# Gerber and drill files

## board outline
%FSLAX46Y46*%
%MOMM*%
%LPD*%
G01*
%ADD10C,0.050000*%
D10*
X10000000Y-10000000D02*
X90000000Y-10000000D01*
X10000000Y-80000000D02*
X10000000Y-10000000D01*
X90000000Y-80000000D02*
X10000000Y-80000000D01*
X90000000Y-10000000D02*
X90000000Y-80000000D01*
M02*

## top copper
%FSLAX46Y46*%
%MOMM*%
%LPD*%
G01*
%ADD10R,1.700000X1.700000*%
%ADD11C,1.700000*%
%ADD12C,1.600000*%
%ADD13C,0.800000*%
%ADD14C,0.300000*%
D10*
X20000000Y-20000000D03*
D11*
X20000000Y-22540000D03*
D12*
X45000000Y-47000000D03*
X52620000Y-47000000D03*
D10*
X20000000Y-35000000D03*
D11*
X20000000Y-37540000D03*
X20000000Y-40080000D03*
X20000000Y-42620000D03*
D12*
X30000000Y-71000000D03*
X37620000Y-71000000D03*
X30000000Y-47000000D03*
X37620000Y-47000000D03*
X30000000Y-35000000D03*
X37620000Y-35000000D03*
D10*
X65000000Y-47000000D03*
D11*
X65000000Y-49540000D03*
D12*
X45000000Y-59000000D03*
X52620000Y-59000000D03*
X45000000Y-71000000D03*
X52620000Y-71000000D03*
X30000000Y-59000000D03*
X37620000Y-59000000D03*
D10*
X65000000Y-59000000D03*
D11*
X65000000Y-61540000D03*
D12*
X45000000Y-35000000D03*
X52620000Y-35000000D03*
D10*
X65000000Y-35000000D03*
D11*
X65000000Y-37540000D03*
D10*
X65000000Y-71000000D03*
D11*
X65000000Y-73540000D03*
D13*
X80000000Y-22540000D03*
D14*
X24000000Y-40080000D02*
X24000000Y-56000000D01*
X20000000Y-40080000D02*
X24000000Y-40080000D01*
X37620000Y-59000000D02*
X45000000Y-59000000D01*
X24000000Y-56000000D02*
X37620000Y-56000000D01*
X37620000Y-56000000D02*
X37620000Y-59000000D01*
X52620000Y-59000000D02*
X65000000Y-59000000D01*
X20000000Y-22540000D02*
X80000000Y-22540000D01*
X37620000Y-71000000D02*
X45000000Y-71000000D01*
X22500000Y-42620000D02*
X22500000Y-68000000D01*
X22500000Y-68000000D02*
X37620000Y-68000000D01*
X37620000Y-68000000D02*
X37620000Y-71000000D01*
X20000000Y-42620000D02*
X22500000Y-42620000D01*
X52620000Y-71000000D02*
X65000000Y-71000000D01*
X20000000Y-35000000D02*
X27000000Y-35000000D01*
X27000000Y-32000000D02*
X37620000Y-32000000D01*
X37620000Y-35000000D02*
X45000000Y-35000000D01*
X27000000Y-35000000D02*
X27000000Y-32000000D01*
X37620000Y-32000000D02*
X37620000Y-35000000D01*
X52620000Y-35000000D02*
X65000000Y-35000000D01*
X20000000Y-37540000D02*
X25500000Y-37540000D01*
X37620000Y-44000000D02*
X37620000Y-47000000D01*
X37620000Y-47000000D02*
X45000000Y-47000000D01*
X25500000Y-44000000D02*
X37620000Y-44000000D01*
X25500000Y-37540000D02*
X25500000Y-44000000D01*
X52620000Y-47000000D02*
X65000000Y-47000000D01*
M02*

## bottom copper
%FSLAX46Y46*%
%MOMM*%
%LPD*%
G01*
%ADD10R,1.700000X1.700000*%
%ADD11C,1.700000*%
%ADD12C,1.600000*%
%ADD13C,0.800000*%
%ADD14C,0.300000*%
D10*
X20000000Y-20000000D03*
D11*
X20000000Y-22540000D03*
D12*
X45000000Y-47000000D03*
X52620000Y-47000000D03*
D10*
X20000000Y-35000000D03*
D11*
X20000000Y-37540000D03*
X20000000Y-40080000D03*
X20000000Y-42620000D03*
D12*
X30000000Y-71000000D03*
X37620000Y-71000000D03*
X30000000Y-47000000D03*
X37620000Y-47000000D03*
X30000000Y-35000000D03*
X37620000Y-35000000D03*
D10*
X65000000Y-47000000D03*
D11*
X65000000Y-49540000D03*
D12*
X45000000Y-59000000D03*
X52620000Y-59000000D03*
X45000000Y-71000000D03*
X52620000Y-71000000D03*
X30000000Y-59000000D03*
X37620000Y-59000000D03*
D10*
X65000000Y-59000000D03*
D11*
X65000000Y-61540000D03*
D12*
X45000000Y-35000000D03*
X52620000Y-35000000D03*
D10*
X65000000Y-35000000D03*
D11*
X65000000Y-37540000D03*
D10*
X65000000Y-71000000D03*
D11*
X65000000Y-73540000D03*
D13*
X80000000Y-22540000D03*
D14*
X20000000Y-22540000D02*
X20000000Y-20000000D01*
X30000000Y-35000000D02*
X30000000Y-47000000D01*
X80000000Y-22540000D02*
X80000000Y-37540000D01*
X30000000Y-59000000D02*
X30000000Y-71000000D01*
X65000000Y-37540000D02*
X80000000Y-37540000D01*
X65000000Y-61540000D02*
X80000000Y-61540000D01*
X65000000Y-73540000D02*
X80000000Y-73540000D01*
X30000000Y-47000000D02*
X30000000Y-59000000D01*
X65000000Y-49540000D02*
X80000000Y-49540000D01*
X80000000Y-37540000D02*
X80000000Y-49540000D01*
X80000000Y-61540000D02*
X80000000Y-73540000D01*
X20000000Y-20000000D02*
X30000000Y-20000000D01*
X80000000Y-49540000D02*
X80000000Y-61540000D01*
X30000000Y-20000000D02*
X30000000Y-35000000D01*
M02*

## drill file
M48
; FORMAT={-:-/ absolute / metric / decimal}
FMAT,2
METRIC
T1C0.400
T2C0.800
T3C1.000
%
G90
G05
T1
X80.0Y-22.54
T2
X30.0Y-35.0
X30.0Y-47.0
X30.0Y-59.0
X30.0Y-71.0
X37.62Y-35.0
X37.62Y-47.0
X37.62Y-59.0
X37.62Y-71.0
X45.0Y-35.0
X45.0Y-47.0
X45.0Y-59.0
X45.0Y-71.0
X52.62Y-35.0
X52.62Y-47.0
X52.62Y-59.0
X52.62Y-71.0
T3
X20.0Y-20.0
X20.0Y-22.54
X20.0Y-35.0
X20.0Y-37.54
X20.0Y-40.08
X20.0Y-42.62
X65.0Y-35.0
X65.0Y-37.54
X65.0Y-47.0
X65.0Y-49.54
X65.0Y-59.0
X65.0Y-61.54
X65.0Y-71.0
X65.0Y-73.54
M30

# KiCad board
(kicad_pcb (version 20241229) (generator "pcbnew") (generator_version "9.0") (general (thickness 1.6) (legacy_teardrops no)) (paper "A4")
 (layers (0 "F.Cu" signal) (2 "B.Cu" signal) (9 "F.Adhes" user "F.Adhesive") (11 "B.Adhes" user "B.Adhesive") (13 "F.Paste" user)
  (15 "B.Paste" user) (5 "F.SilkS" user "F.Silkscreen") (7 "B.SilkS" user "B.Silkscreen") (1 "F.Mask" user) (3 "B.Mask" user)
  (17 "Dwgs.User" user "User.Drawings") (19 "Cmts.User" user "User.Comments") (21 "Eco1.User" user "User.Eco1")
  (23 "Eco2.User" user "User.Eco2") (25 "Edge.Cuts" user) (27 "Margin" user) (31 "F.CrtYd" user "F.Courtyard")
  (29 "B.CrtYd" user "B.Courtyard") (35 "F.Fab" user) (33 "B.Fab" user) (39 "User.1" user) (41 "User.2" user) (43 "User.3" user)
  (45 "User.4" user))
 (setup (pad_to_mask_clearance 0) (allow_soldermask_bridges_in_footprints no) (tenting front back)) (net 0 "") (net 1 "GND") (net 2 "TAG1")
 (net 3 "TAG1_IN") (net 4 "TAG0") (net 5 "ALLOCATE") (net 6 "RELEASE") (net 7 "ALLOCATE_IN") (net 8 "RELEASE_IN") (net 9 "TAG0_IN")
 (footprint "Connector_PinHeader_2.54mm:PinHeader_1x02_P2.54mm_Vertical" (layer "F.Cu") (at 20 20)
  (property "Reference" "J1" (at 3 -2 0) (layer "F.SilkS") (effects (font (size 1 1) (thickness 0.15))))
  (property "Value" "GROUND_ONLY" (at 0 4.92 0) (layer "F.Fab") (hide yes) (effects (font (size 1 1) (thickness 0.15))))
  (pad "1" thru_hole rect (at 0 0) (size 1.7 1.7) (drill 1) (layers "*.Cu" "*.Mask") (remove_unused_layers no) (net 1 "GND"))
  (pad "2" thru_hole circle (at 0 2.54) (size 1.7 1.7) (drill 1) (layers "*.Cu" "*.Mask") (remove_unused_layers no) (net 1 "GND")))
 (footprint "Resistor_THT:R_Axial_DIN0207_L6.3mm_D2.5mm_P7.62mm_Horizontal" (layer "F.Cu") (at 45 47)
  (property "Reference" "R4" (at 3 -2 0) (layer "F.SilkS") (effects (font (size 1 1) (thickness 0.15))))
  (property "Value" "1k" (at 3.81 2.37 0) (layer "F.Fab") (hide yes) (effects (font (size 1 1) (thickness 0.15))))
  (pad "1" thru_hole circle (at 0 0) (size 1.6 1.6) (drill 0.8) (layers "*.Cu" "*.Mask") (remove_unused_layers no) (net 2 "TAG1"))
  (pad "2" thru_hole circle (at 7.62 0) (size 1.6 1.6) (drill 0.8) (layers "*.Cu" "*.Mask") (remove_unused_layers no) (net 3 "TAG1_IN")))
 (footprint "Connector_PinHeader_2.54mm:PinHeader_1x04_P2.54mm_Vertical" (layer "F.Cu") (at 20 35)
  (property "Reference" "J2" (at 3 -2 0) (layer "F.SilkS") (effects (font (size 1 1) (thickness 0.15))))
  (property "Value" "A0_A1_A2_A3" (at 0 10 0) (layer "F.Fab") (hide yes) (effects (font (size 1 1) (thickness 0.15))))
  (pad "1" thru_hole rect (at 0 0) (size 1.7 1.7) (drill 1) (layers "*.Cu" "*.Mask") (remove_unused_layers no) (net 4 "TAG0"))
  (pad "2" thru_hole circle (at 0 2.54) (size 1.7 1.7) (drill 1) (layers "*.Cu" "*.Mask") (remove_unused_layers no) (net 2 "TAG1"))
  (pad "3" thru_hole circle (at 0 5.08) (size 1.7 1.7) (drill 1) (layers "*.Cu" "*.Mask") (remove_unused_layers no) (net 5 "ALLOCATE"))
  (pad "4" thru_hole circle (at 0 7.62) (size 1.7 1.7) (drill 1) (layers "*.Cu" "*.Mask") (remove_unused_layers no) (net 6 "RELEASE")))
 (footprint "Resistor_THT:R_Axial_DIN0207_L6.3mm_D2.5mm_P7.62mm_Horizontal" (layer "F.Cu") (at 30 71)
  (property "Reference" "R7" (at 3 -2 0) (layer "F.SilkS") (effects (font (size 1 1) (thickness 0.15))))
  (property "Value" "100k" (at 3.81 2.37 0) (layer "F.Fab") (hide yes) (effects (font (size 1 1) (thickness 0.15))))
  (pad "1" thru_hole circle (at 0 0) (size 1.6 1.6) (drill 0.8) (layers "*.Cu" "*.Mask") (remove_unused_layers no) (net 1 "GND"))
  (pad "2" thru_hole circle (at 7.62 0) (size 1.6 1.6) (drill 0.8) (layers "*.Cu" "*.Mask") (remove_unused_layers no) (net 6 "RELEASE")))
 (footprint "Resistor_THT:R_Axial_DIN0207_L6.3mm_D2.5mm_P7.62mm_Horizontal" (layer "F.Cu") (at 30 47)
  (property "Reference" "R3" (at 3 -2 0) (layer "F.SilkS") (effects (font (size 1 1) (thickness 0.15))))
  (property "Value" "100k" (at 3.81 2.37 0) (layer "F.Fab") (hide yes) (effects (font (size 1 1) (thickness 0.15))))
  (pad "1" thru_hole circle (at 0 0) (size 1.6 1.6) (drill 0.8) (layers "*.Cu" "*.Mask") (remove_unused_layers no) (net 1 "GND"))
  (pad "2" thru_hole circle (at 7.62 0) (size 1.6 1.6) (drill 0.8) (layers "*.Cu" "*.Mask") (remove_unused_layers no) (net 2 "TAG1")))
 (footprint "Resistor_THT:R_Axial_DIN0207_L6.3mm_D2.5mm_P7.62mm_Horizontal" (layer "F.Cu") (at 30 35)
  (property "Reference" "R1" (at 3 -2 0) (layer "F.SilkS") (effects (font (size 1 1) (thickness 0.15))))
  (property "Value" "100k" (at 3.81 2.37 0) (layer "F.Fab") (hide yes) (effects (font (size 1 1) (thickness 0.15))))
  (pad "1" thru_hole circle (at 0 0) (size 1.6 1.6) (drill 0.8) (layers "*.Cu" "*.Mask") (remove_unused_layers no) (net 1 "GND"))
  (pad "2" thru_hole circle (at 7.62 0) (size 1.6 1.6) (drill 0.8) (layers "*.Cu" "*.Mask") (remove_unused_layers no) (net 4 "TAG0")))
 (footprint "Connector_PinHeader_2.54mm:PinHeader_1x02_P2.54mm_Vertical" (layer "F.Cu") (at 65 47)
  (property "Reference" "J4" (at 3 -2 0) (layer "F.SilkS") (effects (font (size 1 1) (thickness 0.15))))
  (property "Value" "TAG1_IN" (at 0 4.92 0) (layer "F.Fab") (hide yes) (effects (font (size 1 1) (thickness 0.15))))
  (pad "1" thru_hole rect (at 0 0) (size 1.7 1.7) (drill 1) (layers "*.Cu" "*.Mask") (remove_unused_layers no) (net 3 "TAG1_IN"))
  (pad "2" thru_hole circle (at 0 2.54) (size 1.7 1.7) (drill 1) (layers "*.Cu" "*.Mask") (remove_unused_layers no) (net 1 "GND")))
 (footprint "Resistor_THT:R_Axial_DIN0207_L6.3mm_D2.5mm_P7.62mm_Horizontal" (layer "F.Cu") (at 45 59)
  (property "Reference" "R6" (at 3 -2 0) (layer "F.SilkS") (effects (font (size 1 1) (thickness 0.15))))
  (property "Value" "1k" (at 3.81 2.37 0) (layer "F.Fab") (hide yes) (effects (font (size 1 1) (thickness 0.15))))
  (pad "1" thru_hole circle (at 0 0) (size 1.6 1.6) (drill 0.8) (layers "*.Cu" "*.Mask") (remove_unused_layers no) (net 5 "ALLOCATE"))
  (pad "2" thru_hole circle (at 7.62 0) (size 1.6 1.6) (drill 0.8) (layers "*.Cu" "*.Mask") (remove_unused_layers no) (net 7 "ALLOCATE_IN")))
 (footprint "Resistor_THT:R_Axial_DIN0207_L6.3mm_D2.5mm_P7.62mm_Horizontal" (layer "F.Cu") (at 45 71)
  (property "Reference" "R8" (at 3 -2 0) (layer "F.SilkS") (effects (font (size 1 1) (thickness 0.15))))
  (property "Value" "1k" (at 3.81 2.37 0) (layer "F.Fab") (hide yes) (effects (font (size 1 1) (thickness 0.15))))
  (pad "1" thru_hole circle (at 0 0) (size 1.6 1.6) (drill 0.8) (layers "*.Cu" "*.Mask") (remove_unused_layers no) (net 6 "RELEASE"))
  (pad "2" thru_hole circle (at 7.62 0) (size 1.6 1.6) (drill 0.8) (layers "*.Cu" "*.Mask") (remove_unused_layers no) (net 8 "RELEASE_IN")))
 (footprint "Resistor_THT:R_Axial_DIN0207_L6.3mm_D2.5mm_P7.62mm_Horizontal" (layer "F.Cu") (at 30 59)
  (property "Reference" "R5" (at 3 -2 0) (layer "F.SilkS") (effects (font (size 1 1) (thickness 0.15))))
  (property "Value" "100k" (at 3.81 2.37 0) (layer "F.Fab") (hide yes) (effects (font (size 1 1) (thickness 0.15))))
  (pad "1" thru_hole circle (at 0 0) (size 1.6 1.6) (drill 0.8) (layers "*.Cu" "*.Mask") (remove_unused_layers no) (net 1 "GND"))
  (pad "2" thru_hole circle (at 7.62 0) (size 1.6 1.6) (drill 0.8) (layers "*.Cu" "*.Mask") (remove_unused_layers no) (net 5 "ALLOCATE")))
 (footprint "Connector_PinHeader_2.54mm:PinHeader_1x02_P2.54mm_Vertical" (layer "F.Cu") (at 65 59)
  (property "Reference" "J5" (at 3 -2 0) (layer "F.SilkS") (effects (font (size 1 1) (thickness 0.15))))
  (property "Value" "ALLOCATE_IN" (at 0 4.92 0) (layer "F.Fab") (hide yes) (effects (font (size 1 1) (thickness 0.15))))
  (pad "1" thru_hole rect (at 0 0) (size 1.7 1.7) (drill 1) (layers "*.Cu" "*.Mask") (remove_unused_layers no) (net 7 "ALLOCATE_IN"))
  (pad "2" thru_hole circle (at 0 2.54) (size 1.7 1.7) (drill 1) (layers "*.Cu" "*.Mask") (remove_unused_layers no) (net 1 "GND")))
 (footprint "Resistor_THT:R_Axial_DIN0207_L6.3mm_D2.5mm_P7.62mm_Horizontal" (layer "F.Cu") (at 45 35)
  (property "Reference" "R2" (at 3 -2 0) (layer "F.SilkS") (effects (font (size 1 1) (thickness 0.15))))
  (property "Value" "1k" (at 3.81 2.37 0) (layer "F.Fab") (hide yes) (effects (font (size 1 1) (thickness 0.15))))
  (pad "1" thru_hole circle (at 0 0) (size 1.6 1.6) (drill 0.8) (layers "*.Cu" "*.Mask") (remove_unused_layers no) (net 4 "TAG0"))
  (pad "2" thru_hole circle (at 7.62 0) (size 1.6 1.6) (drill 0.8) (layers "*.Cu" "*.Mask") (remove_unused_layers no) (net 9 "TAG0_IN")))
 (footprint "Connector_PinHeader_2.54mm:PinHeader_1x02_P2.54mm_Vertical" (layer "F.Cu") (at 65 35)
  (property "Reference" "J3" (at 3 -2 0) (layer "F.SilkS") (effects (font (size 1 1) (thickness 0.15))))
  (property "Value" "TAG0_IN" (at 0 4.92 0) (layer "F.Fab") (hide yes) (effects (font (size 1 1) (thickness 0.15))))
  (pad "1" thru_hole rect (at 0 0) (size 1.7 1.7) (drill 1) (layers "*.Cu" "*.Mask") (remove_unused_layers no) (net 9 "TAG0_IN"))
  (pad "2" thru_hole circle (at 0 2.54) (size 1.7 1.7) (drill 1) (layers "*.Cu" "*.Mask") (remove_unused_layers no) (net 1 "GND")))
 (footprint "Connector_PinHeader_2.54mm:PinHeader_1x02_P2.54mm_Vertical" (layer "F.Cu") (at 65 71)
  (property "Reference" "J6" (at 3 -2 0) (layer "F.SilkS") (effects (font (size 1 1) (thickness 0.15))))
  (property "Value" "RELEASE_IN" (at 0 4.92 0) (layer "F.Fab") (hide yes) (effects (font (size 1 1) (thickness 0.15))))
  (pad "1" thru_hole rect (at 0 0) (size 1.7 1.7) (drill 1) (layers "*.Cu" "*.Mask") (remove_unused_layers no) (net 8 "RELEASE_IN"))
  (pad "2" thru_hole circle (at 0 2.54) (size 1.7 1.7) (drill 1) (layers "*.Cu" "*.Mask") (remove_unused_layers no) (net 1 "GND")))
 (gr_line (start 10 10) (end 90 10) (stroke (width 0.05) (type default)) (layer "Edge.Cuts"))
 (gr_line (start 10 80) (end 10 10) (stroke (width 0.05) (type default)) (layer "Edge.Cuts"))
 (gr_line (start 90 80) (end 10 80) (stroke (width 0.05) (type default)) (layer "Edge.Cuts"))
 (gr_line (start 90 10) (end 90 80) (stroke (width 0.05) (type default)) (layer "Edge.Cuts"))
 (segment (start 24 40.08) (end 24 56) (width 0.3) (layer "F.Cu") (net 5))
 (segment (start 20 40.08) (end 24 40.08) (width 0.3) (layer "F.Cu") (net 5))
 (segment (start 37.62 59) (end 45 59) (width 0.3) (layer "F.Cu") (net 5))
 (segment (start 24 56) (end 37.62 56) (width 0.3) (layer "F.Cu") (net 5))
 (segment (start 37.62 56) (end 37.62 59) (width 0.3) (layer "F.Cu") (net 5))
 (segment (start 52.62 59) (end 65 59) (width 0.3) (layer "F.Cu") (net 7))
 (segment (start 20 22.54) (end 80 22.54) (width 0.3) (layer "F.Cu") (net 1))
 (via (at 80 22.54) (size 0.8) (drill 0.4) (layers "F.Cu" "B.Cu") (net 1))
 (segment (start 20 22.54) (end 20 20) (width 0.3) (layer "B.Cu") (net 1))
 (segment (start 30 35) (end 30 47) (width 0.3) (layer "B.Cu") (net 1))
 (segment (start 80 22.54) (end 80 37.54) (width 0.3) (layer "B.Cu") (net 1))
 (segment (start 30 59) (end 30 71) (width 0.3) (layer "B.Cu") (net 1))
 (segment (start 65 37.54) (end 80 37.54) (width 0.3) (layer "B.Cu") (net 1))
 (segment (start 65 61.54) (end 80 61.54) (width 0.3) (layer "B.Cu") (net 1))
 (segment (start 65 73.54) (end 80 73.54) (width 0.3) (layer "B.Cu") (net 1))
 (segment (start 30 47) (end 30 59) (width 0.3) (layer "B.Cu") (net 1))
 (segment (start 65 49.54) (end 80 49.54) (width 0.3) (layer "B.Cu") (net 1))
 (segment (start 80 37.54) (end 80 49.54) (width 0.3) (layer "B.Cu") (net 1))
 (segment (start 80 61.54) (end 80 73.54) (width 0.3) (layer "B.Cu") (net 1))
 (segment (start 20 20) (end 30 20) (width 0.3) (layer "B.Cu") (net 1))
 (segment (start 80 49.54) (end 80 61.54) (width 0.3) (layer "B.Cu") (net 1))
 (segment (start 30 20) (end 30 35) (width 0.3) (layer "B.Cu") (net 1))
 (segment (start 37.62 71) (end 45 71) (width 0.3) (layer "F.Cu") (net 6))
 (segment (start 22.5 42.62) (end 22.5 68) (width 0.3) (layer "F.Cu") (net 6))
 (segment (start 22.5 68) (end 37.62 68) (width 0.3) (layer "F.Cu") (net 6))
 (segment (start 37.62 68) (end 37.62 71) (width 0.3) (layer "F.Cu") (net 6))
 (segment (start 20 42.62) (end 22.5 42.62) (width 0.3) (layer "F.Cu") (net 6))
 (segment (start 52.62 71) (end 65 71) (width 0.3) (layer "F.Cu") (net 8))
 (segment (start 20 35) (end 27 35) (width 0.3) (layer "F.Cu") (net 4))
 (segment (start 27 32) (end 37.62 32) (width 0.3) (layer "F.Cu") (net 4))
 (segment (start 37.62 35) (end 45 35) (width 0.3) (layer "F.Cu") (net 4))
 (segment (start 27 35) (end 27 32) (width 0.3) (layer "F.Cu") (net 4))
 (segment (start 37.62 32) (end 37.62 35) (width 0.3) (layer "F.Cu") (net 4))
 (segment (start 52.62 35) (end 65 35) (width 0.3) (layer "F.Cu") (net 9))
 (segment (start 20 37.54) (end 25.5 37.54) (width 0.3) (layer "F.Cu") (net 2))
 (segment (start 37.62 44) (end 37.62 47) (width 0.3) (layer "F.Cu") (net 2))
 (segment (start 37.62 47) (end 45 47) (width 0.3) (layer "F.Cu") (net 2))
 (segment (start 25.5 44) (end 37.62 44) (width 0.3) (layer "F.Cu") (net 2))
 (segment (start 25.5 37.54) (end 25.5 44) (width 0.3) (layer "F.Cu") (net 2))
 (segment (start 52.62 47) (end 65 47) (width 0.3) (layer "F.Cu") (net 3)))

